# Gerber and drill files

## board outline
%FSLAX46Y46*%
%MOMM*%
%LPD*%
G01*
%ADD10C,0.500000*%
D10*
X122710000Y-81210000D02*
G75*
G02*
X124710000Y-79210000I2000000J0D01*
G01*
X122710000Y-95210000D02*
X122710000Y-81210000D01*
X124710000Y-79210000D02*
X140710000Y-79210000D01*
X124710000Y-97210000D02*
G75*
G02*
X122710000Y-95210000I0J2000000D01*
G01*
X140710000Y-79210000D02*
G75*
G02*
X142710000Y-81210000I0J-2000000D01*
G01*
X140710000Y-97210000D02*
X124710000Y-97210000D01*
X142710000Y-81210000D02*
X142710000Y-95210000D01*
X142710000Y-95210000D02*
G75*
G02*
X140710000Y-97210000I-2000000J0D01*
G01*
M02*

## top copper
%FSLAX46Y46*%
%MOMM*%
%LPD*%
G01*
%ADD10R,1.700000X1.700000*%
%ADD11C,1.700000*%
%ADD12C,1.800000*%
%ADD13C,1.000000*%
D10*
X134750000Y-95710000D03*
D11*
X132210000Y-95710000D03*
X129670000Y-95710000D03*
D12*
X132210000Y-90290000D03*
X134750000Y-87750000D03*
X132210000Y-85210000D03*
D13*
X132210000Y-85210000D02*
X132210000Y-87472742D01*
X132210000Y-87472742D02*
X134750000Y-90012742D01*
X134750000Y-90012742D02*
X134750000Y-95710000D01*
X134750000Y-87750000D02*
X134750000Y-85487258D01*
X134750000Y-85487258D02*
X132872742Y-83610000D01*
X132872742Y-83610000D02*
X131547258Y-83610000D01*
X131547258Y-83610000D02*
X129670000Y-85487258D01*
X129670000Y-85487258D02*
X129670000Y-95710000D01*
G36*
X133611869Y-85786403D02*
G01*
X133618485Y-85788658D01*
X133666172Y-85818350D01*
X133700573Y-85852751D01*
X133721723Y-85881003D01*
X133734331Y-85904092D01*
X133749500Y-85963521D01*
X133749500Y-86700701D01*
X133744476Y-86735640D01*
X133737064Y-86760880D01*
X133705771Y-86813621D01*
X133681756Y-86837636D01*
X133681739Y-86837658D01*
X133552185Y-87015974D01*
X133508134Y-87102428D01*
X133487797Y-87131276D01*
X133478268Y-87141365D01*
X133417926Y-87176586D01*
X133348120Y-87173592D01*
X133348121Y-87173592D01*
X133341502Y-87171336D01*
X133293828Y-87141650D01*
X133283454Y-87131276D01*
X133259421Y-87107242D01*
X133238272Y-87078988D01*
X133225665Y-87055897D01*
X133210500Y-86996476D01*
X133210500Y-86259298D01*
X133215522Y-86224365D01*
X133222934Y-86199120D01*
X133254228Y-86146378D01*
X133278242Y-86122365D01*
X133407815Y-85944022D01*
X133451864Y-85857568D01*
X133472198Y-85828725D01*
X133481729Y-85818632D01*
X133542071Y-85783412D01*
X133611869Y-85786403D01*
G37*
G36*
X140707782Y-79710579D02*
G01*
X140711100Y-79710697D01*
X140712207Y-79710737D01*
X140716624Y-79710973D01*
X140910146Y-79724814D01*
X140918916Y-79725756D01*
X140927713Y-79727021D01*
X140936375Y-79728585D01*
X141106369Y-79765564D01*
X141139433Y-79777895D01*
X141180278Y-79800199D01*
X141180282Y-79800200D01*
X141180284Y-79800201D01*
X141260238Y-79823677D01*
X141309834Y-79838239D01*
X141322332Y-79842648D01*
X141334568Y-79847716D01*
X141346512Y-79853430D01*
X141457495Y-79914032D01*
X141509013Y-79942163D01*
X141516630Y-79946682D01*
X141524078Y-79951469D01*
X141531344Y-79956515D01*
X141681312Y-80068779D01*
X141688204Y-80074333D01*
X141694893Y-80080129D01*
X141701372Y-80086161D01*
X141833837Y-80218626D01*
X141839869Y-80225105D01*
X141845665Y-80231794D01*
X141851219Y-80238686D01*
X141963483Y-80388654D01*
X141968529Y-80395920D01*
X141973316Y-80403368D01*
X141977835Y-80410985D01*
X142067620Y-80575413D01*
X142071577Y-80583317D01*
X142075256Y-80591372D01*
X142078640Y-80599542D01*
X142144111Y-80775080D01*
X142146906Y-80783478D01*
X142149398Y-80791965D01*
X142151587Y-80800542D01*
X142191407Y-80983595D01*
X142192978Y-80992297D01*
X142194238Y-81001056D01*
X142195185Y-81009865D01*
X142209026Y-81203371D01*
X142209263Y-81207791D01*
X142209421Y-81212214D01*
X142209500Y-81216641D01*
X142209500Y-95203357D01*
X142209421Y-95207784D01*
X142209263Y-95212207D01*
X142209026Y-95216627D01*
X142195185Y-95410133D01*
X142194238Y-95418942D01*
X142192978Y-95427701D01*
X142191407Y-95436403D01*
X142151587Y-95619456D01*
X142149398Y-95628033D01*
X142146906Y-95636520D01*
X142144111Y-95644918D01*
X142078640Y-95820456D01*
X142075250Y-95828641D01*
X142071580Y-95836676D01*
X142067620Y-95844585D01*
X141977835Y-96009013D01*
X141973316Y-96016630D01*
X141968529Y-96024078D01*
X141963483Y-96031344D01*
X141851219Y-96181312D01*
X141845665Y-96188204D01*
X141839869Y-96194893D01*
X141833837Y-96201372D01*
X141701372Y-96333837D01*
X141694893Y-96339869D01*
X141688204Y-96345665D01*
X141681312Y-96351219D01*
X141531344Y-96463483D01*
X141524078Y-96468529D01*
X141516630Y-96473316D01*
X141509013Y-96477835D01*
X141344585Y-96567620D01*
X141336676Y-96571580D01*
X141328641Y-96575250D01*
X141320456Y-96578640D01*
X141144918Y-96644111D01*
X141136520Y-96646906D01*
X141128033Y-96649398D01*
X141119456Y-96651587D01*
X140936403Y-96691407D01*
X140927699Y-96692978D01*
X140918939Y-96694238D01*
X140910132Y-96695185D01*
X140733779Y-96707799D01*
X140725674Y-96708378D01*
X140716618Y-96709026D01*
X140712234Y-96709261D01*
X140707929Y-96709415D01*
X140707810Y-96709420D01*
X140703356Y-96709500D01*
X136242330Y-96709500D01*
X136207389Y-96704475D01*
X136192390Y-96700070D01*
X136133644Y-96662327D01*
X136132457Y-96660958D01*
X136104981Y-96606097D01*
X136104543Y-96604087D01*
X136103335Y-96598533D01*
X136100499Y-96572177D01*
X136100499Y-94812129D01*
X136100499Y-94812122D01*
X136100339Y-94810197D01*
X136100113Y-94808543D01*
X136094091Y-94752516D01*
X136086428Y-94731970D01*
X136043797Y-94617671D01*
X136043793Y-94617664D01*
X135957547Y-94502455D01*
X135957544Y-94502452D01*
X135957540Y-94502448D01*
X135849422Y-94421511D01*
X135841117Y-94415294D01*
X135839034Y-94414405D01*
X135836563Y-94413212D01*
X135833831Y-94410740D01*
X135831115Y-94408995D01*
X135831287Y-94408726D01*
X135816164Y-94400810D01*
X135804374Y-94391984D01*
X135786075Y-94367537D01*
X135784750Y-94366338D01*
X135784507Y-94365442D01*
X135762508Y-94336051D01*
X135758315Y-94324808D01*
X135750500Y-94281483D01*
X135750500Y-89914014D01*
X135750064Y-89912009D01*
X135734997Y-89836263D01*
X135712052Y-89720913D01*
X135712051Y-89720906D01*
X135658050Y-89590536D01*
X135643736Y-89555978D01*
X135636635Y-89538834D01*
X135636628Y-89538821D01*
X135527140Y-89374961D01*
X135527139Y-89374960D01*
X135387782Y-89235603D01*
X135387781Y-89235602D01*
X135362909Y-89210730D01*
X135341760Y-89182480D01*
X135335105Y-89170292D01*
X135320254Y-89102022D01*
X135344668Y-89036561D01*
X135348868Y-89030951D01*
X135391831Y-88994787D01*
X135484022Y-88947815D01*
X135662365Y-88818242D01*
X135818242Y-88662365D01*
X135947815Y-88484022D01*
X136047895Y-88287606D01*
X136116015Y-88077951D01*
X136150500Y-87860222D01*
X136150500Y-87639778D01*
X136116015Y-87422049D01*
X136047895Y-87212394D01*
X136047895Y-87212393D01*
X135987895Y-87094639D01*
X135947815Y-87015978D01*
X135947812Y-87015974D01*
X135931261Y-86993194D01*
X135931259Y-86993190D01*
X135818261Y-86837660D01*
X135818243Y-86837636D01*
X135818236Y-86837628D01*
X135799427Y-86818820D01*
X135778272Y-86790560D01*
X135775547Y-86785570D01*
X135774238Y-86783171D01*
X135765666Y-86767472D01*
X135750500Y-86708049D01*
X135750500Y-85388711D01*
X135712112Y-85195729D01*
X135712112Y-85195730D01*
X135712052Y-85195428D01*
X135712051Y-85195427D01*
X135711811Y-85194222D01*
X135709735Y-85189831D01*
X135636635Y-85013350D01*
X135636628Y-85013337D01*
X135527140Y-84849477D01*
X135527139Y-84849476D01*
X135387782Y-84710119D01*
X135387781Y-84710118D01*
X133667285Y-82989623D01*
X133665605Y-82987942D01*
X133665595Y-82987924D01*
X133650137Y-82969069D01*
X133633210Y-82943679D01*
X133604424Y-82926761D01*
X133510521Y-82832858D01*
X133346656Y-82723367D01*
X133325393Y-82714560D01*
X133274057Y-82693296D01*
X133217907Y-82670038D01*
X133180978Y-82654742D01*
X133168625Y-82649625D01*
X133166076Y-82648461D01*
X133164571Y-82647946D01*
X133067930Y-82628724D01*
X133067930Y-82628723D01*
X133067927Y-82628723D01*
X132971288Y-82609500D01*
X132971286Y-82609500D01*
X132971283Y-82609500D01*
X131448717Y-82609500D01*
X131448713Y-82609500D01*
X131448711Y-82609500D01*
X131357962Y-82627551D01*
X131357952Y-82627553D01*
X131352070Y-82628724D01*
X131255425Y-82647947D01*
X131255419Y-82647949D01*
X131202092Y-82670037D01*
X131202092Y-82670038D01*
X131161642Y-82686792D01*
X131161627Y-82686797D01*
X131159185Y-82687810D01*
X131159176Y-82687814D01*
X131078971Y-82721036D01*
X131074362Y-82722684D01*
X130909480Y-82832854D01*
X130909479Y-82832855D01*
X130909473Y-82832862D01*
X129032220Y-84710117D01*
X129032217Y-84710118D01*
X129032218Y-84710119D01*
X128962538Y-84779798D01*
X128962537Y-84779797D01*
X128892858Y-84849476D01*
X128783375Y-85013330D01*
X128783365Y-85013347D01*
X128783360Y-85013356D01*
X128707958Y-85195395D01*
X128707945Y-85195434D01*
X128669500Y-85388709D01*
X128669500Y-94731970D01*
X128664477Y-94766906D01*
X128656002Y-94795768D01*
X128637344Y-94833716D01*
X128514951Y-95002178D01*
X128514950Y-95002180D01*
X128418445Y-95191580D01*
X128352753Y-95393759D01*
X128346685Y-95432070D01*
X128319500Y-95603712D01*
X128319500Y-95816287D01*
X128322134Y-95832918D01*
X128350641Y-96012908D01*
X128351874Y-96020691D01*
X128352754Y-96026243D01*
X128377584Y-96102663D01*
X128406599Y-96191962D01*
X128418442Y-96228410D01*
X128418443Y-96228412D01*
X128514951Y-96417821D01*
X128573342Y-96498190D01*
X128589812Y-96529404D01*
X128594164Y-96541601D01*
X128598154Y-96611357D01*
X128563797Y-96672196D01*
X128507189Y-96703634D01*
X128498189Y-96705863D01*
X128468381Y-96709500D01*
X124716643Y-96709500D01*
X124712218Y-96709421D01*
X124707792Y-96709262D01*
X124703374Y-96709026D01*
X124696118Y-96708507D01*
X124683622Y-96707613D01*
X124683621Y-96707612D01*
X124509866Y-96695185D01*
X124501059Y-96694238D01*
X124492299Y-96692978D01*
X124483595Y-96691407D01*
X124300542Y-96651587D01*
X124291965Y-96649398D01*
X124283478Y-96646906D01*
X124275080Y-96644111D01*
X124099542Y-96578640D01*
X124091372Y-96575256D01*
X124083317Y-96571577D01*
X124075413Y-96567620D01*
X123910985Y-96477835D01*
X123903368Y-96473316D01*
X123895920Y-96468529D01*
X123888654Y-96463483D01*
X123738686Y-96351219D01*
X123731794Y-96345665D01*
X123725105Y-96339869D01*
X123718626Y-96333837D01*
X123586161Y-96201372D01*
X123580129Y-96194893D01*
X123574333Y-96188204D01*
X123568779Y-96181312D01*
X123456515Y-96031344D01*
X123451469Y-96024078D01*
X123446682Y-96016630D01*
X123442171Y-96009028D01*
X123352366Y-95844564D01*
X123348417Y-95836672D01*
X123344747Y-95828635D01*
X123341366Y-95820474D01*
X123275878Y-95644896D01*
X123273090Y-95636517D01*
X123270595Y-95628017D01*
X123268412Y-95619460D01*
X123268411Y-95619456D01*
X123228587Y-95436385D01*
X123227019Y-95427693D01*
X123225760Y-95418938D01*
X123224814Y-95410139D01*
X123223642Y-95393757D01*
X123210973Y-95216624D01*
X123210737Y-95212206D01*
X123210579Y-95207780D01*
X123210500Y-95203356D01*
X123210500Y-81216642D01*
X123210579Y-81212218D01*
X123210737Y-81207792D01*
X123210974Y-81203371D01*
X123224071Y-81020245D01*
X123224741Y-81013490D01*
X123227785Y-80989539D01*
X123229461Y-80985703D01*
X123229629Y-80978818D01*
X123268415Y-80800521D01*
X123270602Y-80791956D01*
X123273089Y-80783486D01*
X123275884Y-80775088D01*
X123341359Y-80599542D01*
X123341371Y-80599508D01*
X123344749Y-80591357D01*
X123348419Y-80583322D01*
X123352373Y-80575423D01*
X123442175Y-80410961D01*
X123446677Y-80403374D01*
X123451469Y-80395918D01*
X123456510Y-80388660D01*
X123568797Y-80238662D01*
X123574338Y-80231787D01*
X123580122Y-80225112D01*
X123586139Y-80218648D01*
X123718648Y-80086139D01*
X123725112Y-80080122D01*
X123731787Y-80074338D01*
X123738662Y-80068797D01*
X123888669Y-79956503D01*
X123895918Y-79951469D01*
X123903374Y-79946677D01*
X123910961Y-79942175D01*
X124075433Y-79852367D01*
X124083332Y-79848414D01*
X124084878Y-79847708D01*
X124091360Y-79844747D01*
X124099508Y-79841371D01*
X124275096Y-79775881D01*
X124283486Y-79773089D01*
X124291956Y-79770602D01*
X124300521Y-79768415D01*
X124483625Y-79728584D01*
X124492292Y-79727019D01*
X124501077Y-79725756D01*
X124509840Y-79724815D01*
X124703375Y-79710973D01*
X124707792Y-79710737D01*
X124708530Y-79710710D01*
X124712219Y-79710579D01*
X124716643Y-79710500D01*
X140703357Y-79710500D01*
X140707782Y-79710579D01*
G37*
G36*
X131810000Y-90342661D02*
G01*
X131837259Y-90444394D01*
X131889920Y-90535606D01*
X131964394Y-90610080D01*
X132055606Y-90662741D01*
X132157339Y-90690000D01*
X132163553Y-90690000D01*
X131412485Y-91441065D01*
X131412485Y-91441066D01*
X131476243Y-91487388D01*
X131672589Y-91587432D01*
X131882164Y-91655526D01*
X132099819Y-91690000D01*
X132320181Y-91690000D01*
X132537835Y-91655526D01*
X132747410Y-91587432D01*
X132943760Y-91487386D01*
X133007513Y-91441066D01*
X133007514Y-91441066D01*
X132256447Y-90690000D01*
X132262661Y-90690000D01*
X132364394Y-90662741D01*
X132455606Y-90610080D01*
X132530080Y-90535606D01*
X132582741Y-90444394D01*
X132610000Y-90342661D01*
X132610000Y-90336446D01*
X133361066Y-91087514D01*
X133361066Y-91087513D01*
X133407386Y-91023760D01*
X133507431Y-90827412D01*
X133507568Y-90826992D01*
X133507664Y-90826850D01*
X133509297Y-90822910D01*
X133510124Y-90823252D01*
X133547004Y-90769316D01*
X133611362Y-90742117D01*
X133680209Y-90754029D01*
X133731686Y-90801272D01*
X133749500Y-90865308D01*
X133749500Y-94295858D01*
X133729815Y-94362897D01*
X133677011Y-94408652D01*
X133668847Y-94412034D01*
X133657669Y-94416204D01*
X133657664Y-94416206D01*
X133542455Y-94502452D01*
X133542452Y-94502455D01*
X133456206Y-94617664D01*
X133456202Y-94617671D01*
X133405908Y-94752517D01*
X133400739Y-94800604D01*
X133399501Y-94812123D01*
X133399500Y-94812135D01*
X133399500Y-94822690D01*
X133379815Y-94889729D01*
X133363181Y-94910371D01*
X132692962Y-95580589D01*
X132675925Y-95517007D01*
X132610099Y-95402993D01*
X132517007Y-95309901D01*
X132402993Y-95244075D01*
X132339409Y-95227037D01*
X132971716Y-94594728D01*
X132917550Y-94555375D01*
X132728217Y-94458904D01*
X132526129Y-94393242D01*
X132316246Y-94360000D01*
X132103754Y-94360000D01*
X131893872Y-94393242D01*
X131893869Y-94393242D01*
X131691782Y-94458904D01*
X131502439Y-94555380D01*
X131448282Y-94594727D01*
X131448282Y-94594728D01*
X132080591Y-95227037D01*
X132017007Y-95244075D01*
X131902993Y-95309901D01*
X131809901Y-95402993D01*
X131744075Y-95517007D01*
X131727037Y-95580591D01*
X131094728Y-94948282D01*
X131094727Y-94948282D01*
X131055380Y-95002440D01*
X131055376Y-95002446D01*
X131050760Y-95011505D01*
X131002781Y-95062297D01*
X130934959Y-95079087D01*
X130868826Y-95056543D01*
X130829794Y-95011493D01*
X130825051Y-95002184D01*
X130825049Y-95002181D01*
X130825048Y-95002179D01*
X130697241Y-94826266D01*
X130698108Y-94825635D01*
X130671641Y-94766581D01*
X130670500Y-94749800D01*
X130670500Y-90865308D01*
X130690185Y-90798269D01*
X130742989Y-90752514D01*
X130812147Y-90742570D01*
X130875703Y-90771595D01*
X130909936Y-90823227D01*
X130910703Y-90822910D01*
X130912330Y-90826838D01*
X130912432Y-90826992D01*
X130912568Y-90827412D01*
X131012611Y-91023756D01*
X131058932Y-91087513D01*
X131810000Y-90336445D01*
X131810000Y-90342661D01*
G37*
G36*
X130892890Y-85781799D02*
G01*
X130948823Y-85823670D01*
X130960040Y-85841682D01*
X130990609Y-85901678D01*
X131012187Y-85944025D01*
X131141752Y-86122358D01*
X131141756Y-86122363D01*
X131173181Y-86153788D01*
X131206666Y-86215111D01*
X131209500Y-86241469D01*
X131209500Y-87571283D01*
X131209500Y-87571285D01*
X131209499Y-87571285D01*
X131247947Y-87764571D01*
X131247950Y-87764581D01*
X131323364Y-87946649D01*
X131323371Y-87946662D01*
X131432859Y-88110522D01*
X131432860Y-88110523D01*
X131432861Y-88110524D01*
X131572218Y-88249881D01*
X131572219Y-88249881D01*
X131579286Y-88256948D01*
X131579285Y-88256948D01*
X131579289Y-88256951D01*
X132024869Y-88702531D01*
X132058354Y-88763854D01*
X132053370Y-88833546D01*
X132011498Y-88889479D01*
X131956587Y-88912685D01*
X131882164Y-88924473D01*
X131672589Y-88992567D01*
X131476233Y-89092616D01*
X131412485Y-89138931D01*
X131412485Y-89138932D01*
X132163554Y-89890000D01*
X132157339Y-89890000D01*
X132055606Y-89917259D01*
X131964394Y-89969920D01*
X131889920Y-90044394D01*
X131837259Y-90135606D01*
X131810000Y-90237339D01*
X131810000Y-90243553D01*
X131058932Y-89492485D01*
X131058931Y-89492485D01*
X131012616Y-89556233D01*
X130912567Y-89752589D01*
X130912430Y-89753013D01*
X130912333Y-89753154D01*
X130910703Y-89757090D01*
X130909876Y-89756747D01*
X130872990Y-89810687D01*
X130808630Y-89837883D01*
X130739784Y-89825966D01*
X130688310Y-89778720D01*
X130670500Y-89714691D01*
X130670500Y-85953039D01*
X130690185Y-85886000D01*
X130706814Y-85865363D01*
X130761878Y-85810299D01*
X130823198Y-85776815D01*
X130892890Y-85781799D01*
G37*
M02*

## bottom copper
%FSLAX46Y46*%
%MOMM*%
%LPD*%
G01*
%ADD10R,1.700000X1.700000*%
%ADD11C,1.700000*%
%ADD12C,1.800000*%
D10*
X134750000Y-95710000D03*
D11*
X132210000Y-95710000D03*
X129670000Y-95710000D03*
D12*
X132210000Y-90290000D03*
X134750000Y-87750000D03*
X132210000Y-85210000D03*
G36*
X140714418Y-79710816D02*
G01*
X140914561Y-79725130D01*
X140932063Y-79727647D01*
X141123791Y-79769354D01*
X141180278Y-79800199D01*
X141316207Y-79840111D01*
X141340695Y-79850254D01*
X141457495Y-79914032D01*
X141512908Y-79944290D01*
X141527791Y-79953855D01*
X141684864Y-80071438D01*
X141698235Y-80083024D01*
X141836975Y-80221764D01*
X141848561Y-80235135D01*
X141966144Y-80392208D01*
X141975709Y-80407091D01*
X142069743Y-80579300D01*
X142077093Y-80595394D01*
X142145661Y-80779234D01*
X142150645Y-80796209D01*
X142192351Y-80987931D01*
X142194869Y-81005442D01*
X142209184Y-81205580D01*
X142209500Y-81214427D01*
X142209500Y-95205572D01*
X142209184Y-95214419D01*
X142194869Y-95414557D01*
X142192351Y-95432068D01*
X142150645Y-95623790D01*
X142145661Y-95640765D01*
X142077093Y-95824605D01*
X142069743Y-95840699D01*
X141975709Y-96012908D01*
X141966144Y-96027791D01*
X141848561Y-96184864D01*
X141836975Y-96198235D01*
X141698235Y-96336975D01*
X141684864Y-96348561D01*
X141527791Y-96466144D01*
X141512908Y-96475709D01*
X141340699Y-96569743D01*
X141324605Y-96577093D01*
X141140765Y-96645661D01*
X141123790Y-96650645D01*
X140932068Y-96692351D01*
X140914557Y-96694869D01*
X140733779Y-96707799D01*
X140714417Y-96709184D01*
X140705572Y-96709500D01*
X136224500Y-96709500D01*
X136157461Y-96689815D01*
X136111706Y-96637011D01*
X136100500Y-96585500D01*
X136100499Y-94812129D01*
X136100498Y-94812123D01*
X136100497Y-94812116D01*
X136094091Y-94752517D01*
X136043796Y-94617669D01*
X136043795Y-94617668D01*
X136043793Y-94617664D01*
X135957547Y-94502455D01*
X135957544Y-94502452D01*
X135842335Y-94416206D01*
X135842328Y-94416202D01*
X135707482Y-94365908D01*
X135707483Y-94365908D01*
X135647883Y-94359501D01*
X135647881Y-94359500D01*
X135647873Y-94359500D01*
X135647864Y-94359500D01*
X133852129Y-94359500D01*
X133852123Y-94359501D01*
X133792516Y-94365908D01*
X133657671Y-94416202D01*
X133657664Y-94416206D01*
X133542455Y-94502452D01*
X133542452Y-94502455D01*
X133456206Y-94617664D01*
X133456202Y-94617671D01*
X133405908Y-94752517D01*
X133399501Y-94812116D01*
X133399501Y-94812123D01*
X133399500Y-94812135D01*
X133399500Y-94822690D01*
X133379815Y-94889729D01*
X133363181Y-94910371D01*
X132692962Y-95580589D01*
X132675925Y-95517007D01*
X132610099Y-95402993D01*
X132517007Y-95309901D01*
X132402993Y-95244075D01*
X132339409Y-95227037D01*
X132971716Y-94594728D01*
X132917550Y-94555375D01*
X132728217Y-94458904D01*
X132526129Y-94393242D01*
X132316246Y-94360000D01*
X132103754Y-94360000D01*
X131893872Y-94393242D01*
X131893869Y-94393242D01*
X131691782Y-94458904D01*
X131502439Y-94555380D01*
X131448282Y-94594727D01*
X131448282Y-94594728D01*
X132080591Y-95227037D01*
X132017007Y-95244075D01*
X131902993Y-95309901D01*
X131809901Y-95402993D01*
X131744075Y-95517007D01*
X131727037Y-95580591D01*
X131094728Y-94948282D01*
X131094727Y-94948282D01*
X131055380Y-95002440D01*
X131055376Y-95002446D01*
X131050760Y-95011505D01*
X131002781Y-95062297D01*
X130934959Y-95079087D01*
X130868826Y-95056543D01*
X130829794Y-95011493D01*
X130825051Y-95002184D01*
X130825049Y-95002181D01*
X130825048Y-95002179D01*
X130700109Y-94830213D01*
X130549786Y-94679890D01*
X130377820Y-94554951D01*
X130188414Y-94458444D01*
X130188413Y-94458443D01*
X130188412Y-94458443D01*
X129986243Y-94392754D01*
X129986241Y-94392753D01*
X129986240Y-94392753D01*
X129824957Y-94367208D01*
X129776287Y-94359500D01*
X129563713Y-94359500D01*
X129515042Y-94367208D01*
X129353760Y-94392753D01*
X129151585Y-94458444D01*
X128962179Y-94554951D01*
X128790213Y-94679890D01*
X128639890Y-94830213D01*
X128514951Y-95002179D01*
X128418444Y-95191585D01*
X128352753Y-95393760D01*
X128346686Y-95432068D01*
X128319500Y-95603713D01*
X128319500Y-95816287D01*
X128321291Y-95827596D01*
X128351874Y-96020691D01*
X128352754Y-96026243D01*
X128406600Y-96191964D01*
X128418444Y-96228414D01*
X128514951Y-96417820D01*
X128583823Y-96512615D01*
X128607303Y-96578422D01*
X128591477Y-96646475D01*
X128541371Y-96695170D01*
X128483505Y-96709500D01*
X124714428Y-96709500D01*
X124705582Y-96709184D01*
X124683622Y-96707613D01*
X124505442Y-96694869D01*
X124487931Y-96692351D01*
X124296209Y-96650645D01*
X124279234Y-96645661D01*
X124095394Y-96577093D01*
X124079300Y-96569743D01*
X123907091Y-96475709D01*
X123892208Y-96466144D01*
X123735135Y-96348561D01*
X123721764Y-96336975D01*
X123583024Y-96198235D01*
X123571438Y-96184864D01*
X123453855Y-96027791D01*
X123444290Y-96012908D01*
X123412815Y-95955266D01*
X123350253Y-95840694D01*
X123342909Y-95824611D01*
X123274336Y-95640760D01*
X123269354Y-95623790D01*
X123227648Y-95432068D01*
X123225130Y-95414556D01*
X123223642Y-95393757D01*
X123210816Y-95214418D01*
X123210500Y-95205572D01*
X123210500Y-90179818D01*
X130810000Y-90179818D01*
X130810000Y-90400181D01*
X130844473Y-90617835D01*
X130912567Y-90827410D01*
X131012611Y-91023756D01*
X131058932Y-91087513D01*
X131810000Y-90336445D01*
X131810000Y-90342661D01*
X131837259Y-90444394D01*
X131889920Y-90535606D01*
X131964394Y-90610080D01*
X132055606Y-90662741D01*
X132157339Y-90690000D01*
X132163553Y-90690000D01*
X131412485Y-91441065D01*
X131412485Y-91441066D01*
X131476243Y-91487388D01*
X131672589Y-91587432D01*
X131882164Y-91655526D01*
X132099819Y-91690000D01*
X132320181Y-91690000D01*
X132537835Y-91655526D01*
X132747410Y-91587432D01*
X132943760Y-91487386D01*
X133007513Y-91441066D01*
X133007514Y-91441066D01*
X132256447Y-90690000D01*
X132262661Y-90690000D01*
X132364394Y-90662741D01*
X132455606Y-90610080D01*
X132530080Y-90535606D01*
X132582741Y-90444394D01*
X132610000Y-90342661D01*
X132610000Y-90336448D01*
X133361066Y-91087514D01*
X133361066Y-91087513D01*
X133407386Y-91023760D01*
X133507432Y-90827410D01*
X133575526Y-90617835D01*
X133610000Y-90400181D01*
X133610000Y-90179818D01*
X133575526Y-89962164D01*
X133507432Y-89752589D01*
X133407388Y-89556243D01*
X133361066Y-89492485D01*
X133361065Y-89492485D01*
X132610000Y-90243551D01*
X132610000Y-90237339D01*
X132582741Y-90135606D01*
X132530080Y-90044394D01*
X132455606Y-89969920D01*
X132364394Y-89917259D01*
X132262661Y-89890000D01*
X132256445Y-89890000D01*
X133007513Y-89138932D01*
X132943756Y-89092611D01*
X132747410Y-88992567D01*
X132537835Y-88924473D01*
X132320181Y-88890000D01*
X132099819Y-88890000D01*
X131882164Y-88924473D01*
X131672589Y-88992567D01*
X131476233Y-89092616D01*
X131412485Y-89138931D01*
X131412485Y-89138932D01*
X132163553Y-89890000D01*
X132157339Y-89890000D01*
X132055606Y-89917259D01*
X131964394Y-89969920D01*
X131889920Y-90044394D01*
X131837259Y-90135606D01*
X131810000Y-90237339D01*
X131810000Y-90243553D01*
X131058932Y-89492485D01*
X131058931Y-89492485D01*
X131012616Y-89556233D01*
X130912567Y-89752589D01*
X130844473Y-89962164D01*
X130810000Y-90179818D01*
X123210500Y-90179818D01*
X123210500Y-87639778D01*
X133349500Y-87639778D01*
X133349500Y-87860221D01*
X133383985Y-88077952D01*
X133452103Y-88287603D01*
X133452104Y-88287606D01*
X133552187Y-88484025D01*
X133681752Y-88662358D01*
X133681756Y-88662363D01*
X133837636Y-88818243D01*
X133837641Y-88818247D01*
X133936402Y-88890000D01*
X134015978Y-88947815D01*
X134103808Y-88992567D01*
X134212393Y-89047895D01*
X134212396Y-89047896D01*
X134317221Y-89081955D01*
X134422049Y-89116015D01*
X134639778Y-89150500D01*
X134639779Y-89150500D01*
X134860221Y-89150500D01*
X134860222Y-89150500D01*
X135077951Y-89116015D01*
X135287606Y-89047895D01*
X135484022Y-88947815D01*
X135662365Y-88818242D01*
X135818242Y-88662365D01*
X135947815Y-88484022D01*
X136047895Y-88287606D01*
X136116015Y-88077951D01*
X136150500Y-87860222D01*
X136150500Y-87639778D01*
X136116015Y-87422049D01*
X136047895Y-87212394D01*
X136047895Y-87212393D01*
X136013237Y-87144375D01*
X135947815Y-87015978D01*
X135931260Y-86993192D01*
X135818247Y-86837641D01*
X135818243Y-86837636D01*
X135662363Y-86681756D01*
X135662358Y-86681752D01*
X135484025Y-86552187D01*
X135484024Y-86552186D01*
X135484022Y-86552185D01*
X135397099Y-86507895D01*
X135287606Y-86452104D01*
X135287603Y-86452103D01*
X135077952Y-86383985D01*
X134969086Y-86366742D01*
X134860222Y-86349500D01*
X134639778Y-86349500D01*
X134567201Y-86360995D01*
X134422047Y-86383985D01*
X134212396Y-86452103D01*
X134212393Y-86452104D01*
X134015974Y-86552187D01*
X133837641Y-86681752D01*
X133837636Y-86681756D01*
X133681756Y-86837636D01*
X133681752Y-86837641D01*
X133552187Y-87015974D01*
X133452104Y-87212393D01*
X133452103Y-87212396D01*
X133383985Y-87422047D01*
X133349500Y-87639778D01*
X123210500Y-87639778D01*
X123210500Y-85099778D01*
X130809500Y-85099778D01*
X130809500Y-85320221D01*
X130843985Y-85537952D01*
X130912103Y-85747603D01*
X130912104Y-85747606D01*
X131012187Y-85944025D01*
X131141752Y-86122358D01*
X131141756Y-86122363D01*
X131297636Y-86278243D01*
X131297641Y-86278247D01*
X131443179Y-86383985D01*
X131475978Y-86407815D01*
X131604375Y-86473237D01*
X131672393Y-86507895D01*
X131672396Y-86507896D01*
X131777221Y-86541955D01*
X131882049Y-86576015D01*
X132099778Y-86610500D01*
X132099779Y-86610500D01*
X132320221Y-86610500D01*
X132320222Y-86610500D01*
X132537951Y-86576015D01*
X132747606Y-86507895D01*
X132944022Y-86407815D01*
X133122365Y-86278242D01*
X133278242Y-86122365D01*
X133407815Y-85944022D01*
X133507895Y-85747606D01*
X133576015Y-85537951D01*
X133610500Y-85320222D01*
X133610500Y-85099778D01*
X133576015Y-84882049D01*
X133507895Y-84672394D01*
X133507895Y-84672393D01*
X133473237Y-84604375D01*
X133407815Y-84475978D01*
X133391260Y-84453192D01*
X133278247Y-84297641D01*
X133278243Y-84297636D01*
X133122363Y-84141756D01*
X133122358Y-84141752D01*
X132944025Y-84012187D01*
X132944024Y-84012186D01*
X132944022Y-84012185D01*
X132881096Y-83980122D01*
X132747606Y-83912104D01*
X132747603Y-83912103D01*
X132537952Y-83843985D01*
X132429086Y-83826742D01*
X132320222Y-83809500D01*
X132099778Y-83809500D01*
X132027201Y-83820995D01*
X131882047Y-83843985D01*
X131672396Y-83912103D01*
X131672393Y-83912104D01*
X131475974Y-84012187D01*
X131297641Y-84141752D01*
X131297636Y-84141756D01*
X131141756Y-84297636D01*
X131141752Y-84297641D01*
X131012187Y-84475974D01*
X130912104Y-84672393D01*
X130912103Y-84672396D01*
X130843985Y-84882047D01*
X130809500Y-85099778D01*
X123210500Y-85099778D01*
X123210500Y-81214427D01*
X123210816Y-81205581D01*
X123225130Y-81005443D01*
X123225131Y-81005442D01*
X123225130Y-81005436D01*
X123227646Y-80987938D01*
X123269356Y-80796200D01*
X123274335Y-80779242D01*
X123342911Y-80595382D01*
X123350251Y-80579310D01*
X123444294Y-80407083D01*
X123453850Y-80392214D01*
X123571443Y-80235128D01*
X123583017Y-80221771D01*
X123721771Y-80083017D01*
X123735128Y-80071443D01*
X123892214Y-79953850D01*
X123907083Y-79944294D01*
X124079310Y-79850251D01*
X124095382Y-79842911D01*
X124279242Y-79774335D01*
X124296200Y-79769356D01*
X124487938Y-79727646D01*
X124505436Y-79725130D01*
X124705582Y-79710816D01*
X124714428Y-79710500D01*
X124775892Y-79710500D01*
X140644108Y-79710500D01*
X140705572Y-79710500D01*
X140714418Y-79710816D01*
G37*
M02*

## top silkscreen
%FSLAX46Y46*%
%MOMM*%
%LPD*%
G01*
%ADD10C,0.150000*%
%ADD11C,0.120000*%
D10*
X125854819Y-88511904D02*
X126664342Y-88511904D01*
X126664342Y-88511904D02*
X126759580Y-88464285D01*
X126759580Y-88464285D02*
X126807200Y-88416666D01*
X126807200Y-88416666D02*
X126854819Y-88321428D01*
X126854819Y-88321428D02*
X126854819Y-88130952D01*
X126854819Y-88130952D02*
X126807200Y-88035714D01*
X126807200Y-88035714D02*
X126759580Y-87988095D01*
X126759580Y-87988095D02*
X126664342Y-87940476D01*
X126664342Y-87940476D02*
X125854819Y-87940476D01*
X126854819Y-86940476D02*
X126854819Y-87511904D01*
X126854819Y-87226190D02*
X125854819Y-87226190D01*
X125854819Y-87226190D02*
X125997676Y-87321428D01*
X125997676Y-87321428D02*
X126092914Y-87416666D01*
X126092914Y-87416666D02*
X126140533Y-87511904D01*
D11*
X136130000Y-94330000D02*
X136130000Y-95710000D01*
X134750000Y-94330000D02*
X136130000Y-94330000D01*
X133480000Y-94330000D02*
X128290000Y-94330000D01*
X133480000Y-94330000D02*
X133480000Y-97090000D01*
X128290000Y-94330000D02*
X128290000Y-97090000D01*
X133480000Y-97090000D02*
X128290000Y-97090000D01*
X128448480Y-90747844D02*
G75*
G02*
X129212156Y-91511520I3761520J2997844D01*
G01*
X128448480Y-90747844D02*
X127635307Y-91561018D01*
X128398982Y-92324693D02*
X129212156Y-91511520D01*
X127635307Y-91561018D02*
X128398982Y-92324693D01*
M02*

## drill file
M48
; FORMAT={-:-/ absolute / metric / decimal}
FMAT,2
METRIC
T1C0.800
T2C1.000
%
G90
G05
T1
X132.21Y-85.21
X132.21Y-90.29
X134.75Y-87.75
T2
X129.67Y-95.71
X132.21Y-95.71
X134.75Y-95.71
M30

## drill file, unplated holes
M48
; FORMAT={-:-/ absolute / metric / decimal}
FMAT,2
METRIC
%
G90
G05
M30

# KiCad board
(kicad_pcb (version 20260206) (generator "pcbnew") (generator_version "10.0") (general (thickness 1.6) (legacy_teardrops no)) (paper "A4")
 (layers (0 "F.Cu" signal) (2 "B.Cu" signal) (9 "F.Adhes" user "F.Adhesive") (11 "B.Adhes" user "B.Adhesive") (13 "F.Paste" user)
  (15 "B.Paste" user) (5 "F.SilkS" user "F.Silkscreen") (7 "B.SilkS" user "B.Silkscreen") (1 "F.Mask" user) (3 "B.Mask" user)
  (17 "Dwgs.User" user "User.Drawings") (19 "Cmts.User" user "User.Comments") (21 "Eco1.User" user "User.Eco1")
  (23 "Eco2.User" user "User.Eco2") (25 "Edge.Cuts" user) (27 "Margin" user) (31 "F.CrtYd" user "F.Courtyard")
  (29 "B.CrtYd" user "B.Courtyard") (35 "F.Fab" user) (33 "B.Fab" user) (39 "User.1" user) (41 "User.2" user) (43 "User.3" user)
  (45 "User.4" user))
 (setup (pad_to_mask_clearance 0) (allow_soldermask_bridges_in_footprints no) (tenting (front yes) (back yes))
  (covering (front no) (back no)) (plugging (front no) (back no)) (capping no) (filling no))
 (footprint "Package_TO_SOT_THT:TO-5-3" (layer "F.Cu") (at 132.21 90.29 90)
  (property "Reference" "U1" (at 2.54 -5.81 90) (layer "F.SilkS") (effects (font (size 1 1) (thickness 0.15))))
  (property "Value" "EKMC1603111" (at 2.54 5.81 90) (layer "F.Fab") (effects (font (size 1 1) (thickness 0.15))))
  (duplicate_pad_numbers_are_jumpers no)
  (fp_line (start -1.271018 -4.574693) (end -2.034693 -3.811018) (stroke (width 0.12) (type solid)) (layer "F.SilkS"))
  (fp_line (start -2.034693 -3.811018) (end -1.22152 -2.997844) (stroke (width 0.12) (type solid)) (layer "F.SilkS"))
  (fp_line (start -0.457844 -3.76152) (end -1.271018 -4.574693) (stroke (width 0.12) (type solid)) (layer "F.SilkS"))
  (fp_arc (start -0.457844 -3.76152) (mid 5.941184 3.401184) (end -1.22152 -2.997844) (stroke (width 0.12) (type solid)) (layer "F.SilkS"))
  (pad "1" thru_hole circle (at 5.08 0 90) (size 1.8 1.8) (drill 0.8) (layers "*.Cu" "*.Mask") (remove_unused_layers no) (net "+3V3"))
  (pad "2" thru_hole circle (at 2.54 2.54 90) (size 1.8 1.8) (drill 0.8) (layers "*.Cu" "*.Mask") (remove_unused_layers no) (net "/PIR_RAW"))
  (pad "3" thru_hole circle (at 0 0 90) (size 1.8 1.8) (drill 0.8) (layers "*.Cu" "*.Mask") (remove_unused_layers no) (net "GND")))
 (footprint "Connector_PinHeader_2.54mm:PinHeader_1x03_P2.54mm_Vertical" (layer "F.Cu") (at 134.75 95.71 -90)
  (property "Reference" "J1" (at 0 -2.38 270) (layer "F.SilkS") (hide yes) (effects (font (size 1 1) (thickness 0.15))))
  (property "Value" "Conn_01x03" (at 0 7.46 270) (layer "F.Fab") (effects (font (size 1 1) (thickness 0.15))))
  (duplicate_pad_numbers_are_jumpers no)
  (fp_line (start -1.38 6.46) (end 1.38 6.46) (stroke (width 0.12) (type solid)) (layer "F.SilkS"))
  (fp_line (start -1.38 1.27) (end -1.38 6.46) (stroke (width 0.12) (type solid)) (layer "F.SilkS"))
  (fp_line (start -1.38 1.27) (end 1.38 1.27) (stroke (width 0.12) (type solid)) (layer "F.SilkS"))
  (fp_line (start 1.38 1.27) (end 1.38 6.46) (stroke (width 0.12) (type solid)) (layer "F.SilkS"))
  (fp_line (start -1.38 0) (end -1.38 -1.38) (stroke (width 0.12) (type solid)) (layer "F.SilkS"))
  (fp_line (start -1.38 -1.38) (end 0 -1.38) (stroke (width 0.12) (type solid)) (layer "F.SilkS"))
  (pad "1" thru_hole rect (at 0 0 270) (size 1.7 1.7) (drill 1) (layers "*.Cu" "*.Mask") (remove_unused_layers no) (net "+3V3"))
  (pad "2" thru_hole circle (at 0 2.54 270) (size 1.7 1.7) (drill 1) (layers "*.Cu" "*.Mask") (remove_unused_layers no) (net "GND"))
  (pad "3" thru_hole circle (at 0 5.08 270) (size 1.7 1.7) (drill 1) (layers "*.Cu" "*.Mask") (remove_unused_layers no) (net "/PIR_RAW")))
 (gr_arc (start 122.71 81.21) (mid 123.295786 79.795786) (end 124.71 79.21) (stroke (width 0.5) (type default)) (layer "Edge.Cuts"))
 (gr_line (start 122.71 95.21) (end 122.71 81.21) (stroke (width 0.5) (type default)) (layer "Edge.Cuts"))
 (gr_line (start 124.71 79.21) (end 140.71 79.21) (stroke (width 0.5) (type default)) (layer "Edge.Cuts"))
 (gr_arc (start 124.71 97.21) (mid 123.295786 96.624214) (end 122.71 95.21) (stroke (width 0.5) (type default)) (layer "Edge.Cuts"))
 (gr_arc (start 140.71 79.21) (mid 142.124214 79.795786) (end 142.71 81.21) (stroke (width 0.5) (type default)) (layer "Edge.Cuts"))
 (gr_line (start 140.71 97.21) (end 124.71 97.21) (stroke (width 0.5) (type default)) (layer "Edge.Cuts"))
 (gr_line (start 142.71 81.21) (end 142.71 95.21) (stroke (width 0.5) (type default)) (layer "Edge.Cuts"))
 (gr_arc (start 142.71 95.21) (mid 142.124214 96.624214) (end 140.71 97.21) (stroke (width 0.5) (type default)) (layer "Edge.Cuts"))
 (segment (start 132.21 85.21) (end 132.21 87.472742) (width 1) (layer "F.Cu") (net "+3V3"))
 (segment (start 134.75 90.012742) (end 134.75 95.71) (width 1) (layer "F.Cu") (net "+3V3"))
 (segment (start 132.21 87.472742) (end 134.75 90.012742) (width 1) (layer "F.Cu") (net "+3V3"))
 (segment (start 132.872742 83.61) (end 131.547258 83.61) (width 1) (layer "F.Cu") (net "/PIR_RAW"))
 (segment (start 131.547258 83.61) (end 129.67 85.487258) (width 1) (layer "F.Cu") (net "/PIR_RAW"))
 (segment (start 134.75 85.487258) (end 132.872742 83.61) (width 1) (layer "F.Cu") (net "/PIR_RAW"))
 (segment (start 134.75 87.75) (end 134.75 85.487258) (width 1) (layer "F.Cu") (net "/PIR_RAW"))
 (segment (start 129.67 85.487258) (end 129.67 95.71) (width 1) (layer "F.Cu") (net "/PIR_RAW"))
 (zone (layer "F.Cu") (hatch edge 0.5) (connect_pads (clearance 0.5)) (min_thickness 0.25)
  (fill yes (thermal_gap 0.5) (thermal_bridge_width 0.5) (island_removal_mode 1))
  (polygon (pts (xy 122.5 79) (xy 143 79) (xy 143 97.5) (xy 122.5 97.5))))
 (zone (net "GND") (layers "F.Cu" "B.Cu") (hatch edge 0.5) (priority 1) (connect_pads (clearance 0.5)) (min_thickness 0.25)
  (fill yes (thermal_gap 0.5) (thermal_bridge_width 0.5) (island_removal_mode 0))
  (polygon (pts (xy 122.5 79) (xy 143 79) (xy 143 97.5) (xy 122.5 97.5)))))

